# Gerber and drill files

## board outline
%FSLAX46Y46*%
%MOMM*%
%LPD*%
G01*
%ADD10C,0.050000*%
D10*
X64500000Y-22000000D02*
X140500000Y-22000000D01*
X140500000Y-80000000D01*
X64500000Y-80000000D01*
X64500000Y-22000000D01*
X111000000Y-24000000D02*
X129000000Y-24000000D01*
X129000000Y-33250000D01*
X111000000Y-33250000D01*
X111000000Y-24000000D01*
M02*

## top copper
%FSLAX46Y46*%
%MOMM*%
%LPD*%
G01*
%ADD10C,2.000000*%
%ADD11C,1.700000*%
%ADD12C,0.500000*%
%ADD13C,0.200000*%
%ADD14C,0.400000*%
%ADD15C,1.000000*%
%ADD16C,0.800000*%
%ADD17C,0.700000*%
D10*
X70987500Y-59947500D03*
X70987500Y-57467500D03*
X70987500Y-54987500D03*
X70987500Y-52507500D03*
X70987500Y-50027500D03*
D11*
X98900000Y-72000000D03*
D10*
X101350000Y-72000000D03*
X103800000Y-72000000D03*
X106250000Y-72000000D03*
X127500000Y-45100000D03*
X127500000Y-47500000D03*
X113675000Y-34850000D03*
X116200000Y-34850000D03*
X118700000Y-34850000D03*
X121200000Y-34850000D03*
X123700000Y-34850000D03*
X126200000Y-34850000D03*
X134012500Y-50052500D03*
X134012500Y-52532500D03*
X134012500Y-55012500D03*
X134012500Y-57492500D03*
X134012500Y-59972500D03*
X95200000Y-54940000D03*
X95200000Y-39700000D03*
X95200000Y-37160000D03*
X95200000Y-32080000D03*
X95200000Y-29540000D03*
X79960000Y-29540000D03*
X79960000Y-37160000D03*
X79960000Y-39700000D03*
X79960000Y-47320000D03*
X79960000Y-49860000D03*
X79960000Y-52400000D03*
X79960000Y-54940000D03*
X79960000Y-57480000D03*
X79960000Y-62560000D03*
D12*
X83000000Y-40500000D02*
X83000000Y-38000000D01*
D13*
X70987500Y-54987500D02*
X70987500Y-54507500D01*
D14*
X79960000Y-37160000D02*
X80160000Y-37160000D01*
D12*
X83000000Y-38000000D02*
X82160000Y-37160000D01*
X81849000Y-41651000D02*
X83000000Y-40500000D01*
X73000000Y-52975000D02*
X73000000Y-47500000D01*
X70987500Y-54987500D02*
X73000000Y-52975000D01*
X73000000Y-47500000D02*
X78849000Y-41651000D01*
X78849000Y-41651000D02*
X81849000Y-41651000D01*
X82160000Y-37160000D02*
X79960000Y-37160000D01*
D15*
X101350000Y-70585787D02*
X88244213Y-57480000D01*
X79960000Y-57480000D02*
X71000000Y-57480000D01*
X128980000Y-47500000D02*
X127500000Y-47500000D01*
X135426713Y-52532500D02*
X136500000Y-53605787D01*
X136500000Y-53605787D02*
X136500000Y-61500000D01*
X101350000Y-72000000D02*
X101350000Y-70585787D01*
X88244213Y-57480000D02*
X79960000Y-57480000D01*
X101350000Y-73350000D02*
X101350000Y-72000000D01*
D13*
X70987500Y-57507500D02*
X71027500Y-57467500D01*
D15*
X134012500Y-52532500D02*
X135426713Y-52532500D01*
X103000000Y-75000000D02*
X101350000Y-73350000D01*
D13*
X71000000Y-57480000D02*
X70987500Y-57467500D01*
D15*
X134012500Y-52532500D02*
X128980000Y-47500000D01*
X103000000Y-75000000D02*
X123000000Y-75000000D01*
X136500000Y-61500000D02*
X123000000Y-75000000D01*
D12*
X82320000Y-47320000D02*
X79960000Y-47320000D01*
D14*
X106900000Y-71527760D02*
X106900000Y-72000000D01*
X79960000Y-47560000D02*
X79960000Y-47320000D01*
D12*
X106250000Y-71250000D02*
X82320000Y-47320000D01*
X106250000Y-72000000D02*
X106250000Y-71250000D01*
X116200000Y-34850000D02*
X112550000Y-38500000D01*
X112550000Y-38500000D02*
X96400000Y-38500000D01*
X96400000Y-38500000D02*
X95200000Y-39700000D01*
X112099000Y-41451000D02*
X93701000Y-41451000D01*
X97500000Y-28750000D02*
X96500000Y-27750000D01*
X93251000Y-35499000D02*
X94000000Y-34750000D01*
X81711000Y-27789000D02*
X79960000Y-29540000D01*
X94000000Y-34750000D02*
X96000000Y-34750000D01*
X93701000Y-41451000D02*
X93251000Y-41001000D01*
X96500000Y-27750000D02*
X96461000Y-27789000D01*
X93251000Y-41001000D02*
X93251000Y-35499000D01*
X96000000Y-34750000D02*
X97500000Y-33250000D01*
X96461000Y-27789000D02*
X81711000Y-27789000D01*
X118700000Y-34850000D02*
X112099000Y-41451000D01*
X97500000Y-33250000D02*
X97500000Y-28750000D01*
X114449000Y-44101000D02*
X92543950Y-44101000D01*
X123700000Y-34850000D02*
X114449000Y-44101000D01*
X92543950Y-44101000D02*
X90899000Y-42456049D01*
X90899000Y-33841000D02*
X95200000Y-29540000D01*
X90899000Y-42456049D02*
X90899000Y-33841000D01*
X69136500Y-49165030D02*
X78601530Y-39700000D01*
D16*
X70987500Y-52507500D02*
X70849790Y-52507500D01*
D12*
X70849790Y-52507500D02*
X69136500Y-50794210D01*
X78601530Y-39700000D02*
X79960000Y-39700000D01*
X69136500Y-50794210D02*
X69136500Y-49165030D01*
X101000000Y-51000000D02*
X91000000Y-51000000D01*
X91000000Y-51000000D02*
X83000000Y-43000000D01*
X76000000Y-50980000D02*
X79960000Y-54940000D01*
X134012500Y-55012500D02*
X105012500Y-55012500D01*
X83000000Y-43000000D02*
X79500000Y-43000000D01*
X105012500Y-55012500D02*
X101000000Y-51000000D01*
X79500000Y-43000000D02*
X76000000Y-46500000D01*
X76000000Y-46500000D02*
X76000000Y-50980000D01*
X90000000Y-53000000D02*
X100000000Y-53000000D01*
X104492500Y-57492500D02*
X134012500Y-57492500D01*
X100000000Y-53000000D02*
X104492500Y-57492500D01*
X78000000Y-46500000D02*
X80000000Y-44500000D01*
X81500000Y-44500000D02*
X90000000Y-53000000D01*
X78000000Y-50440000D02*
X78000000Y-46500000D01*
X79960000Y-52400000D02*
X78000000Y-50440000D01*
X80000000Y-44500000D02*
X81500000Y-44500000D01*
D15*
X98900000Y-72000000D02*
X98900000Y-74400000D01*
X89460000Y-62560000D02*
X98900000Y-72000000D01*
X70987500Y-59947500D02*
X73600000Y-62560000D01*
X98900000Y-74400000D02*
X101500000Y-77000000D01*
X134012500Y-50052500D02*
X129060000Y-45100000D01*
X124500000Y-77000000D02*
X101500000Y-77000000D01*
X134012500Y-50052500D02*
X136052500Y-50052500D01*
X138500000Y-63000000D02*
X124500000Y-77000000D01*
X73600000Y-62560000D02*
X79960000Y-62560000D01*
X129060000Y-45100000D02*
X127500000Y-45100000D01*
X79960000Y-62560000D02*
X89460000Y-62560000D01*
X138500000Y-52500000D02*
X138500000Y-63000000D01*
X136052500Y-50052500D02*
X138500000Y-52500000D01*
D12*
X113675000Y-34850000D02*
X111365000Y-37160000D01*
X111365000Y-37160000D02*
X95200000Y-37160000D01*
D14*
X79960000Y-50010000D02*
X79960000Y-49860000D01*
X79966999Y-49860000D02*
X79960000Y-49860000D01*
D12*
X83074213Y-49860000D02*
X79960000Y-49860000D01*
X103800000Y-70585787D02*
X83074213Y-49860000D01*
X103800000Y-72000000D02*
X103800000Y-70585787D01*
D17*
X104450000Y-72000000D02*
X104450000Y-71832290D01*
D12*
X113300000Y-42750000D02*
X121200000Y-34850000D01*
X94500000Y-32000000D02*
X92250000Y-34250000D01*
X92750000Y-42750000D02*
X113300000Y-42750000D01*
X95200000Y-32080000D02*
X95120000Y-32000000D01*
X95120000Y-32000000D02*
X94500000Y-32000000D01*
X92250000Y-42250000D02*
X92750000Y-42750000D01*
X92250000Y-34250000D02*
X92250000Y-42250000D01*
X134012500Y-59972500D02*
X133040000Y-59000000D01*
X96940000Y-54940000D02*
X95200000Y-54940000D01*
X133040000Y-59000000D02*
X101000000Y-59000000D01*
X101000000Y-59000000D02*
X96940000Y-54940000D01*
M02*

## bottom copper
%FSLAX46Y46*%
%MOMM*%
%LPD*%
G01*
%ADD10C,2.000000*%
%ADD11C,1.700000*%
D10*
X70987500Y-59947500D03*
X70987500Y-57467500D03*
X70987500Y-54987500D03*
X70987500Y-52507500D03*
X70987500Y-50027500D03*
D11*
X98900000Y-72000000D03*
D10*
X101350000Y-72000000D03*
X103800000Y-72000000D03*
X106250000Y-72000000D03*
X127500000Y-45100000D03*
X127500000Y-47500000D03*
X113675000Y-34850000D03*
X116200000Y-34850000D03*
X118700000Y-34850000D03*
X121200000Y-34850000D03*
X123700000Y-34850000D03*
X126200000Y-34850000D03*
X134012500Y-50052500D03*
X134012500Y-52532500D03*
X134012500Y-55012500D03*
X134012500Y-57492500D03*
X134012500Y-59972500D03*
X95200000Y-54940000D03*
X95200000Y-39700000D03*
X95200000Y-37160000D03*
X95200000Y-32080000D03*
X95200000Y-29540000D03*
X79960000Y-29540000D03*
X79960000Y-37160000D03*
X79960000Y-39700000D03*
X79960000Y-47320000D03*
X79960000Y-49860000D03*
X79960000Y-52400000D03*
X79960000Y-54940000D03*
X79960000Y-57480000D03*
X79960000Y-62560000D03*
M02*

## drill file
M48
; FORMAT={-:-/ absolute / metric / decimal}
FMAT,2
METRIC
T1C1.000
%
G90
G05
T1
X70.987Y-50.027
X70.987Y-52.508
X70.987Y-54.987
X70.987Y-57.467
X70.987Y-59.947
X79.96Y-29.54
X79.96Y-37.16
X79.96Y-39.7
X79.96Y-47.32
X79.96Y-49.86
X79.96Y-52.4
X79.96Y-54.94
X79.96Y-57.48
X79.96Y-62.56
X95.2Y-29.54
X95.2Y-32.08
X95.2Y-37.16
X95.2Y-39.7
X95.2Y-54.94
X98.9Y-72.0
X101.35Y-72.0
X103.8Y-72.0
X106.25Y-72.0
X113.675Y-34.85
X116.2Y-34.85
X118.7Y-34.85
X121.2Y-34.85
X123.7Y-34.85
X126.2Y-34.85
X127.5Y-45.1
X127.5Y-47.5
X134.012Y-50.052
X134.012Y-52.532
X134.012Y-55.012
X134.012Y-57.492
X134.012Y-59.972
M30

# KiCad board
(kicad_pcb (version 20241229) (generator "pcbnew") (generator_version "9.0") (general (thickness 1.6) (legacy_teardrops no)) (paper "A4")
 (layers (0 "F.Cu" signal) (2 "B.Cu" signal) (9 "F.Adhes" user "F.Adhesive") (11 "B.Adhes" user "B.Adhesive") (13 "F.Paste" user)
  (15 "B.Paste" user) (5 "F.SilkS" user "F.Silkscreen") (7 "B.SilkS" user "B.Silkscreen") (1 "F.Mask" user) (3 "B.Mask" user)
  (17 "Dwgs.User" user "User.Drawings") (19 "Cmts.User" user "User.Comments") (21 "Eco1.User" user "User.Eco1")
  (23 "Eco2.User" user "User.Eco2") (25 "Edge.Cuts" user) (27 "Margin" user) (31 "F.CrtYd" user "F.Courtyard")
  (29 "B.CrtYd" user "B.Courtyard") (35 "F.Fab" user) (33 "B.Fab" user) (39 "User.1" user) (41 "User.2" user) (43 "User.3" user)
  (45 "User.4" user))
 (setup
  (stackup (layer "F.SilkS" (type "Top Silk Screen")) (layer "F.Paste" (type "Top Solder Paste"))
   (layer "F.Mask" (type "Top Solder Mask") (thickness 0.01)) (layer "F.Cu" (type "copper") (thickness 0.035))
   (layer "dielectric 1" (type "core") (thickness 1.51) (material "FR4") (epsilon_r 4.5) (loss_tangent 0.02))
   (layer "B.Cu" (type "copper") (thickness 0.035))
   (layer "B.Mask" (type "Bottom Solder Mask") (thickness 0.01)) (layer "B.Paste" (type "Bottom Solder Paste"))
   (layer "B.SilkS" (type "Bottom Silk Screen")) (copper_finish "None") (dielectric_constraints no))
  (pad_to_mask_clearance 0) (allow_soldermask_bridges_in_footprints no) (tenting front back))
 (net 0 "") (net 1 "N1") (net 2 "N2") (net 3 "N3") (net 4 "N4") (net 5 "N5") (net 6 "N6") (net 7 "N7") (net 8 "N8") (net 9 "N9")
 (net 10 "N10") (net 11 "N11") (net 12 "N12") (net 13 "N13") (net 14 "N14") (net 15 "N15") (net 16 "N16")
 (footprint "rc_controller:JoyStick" (layer "F.Cu") (at 72.1875 61.1875 180)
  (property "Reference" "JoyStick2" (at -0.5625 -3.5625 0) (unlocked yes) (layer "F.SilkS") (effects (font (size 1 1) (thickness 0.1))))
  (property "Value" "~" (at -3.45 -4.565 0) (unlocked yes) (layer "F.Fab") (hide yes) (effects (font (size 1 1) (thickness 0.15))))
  (pad "1" thru_hole circle (at 1.2 1.24 180) (size 2 2) (drill 1) (layers "*.Cu" "*.Mask") (remove_unused_layers no) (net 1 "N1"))
  (pad "2" thru_hole circle (at 1.2 3.72 180) (size 2 2) (drill 1) (layers "*.Cu" "*.Mask") (remove_unused_layers no) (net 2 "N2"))
  (pad "3" thru_hole circle (at 1.2 6.2 180) (size 2 2) (drill 1) (layers "*.Cu" "*.Mask") (remove_unused_layers no) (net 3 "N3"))
  (pad "4" thru_hole circle (at 1.2 8.68 180) (size 2 2) (drill 1) (layers "*.Cu" "*.Mask") (remove_unused_layers no) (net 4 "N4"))
  (pad "5" thru_hole circle (at 1.2 11.16 180) (size 2 2) (drill 1) (layers "*.Cu" "*.Mask") (remove_unused_layers no) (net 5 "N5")))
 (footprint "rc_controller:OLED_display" (layer "F.Cu") (at 97.675 73.2 90)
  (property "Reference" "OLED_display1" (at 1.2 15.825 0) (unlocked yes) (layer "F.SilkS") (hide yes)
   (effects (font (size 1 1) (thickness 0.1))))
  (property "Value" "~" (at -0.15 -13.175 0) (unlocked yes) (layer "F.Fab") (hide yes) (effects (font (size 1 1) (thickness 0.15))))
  (pad "1" thru_hole circle (at 1.2 1.225 90) (size 1.7 1.7) (drill 1) (layers "*.Cu" "*.Mask") (remove_unused_layers no) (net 1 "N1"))
  (pad "2" thru_hole circle (at 1.2 3.675 90) (size 2 2) (drill 1) (layers "*.Cu" "*.Mask") (remove_unused_layers no) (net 2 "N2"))
  (pad "3" thru_hole circle (at 1.2 6.125 90) (size 2 2) (drill 1) (layers "*.Cu" "F.Mask") (remove_unused_layers no) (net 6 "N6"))
  (pad "4" thru_hole circle (at 1.2 8.575 90) (size 2 2) (drill 1) (layers "*.Cu" "*.Mask") (remove_unused_layers no) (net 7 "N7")))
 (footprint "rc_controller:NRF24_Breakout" (layer "F.Cu") (at 110.65 24.1)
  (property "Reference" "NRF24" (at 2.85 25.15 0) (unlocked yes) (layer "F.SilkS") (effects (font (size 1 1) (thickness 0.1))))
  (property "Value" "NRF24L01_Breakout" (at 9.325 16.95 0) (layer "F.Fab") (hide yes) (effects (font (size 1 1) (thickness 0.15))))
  (pad "1" thru_hole circle (at 16.85 21) (size 2 2) (drill 1) (layers "*.Cu" "*.Mask") (remove_unused_layers no) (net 1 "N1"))
  (pad "2" thru_hole circle (at 16.85 23.4) (size 2 2) (drill 1) (layers "*.Cu" "*.Mask") (remove_unused_layers no) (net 2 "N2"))
  (pad "3" thru_hole circle (at 3.025 10.75) (size 2 2) (drill 1) (layers "*.Cu" "*.Mask") (remove_unused_layers no) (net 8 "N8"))
  (pad "4" thru_hole circle (at 5.55 10.75) (size 2 2) (drill 1) (layers "*.Cu" "*.Mask") (remove_unused_layers no) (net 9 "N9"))
  (pad "5" thru_hole circle (at 8.05 10.75) (size 2 2) (drill 1) (layers "*.Cu" "*.Mask") (remove_unused_layers no) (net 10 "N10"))
  (pad "6" thru_hole circle (at 10.55 10.75) (size 2 2) (drill 1) (layers "*.Cu" "*.Mask") (remove_unused_layers no) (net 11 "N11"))
  (pad "7" thru_hole circle (at 13.05 10.75) (size 2 2) (drill 1) (layers "*.Cu" "*.Mask") (remove_unused_layers no) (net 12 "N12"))
  (pad "8" thru_hole circle (at 15.55 10.75) (size 2 2) (drill 1) (layers "*.Cu" "*.Mask") (remove_unused_layers no) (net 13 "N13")))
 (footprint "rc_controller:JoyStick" (layer "F.Cu") (at 132.8125 48.8125)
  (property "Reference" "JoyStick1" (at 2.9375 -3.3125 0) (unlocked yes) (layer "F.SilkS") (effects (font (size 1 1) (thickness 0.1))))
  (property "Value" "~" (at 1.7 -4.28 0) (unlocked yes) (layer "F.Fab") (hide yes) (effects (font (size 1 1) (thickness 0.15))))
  (pad "1" thru_hole circle (at 1.2 1.24) (size 2 2) (drill 1) (layers "*.Cu" "*.Mask") (remove_unused_layers no) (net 1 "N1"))
  (pad "2" thru_hole circle (at 1.2 3.72) (size 2 2) (drill 1) (layers "*.Cu" "*.Mask") (remove_unused_layers no) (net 2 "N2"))
  (pad "3" thru_hole circle (at 1.2 6.2) (size 2 2) (drill 1) (layers "*.Cu" "*.Mask") (remove_unused_layers no) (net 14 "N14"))
  (pad "4" thru_hole circle (at 1.2 8.68) (size 2 2) (drill 1) (layers "*.Cu" "*.Mask") (remove_unused_layers no) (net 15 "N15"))
  (pad "5" thru_hole circle (at 1.2 11.16) (size 2 2) (drill 1) (layers "*.Cu" "*.Mask") (remove_unused_layers no) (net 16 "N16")))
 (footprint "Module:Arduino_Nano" (layer "F.Cu") (at 80 27)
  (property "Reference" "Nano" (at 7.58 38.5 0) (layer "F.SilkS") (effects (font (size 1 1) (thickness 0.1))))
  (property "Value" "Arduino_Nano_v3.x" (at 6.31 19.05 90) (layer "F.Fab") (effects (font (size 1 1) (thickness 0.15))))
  (pad "5" thru_hole circle (at 15.2 27.94 180) (size 2 2) (drill 1) (layers "*.Cu" "*.Mask") (remove_unused_layers no) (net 16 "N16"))
  (pad "11" thru_hole circle (at 15.2 12.7 180) (size 2 2) (drill 1) (layers "*.Cu" "*.Mask") (remove_unused_layers no) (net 9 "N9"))
  (pad "12" thru_hole circle (at 15.2 10.16 180) (size 2 2) (drill 1) (layers "*.Cu" "*.Mask") (remove_unused_layers no) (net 8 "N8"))
  (pad "14" thru_hole circle (at 15.2 5.08 180) (size 2 2) (drill 1) (layers "*.Cu" "*.Mask") (remove_unused_layers no) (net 11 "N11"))
  (pad "15" thru_hole circle (at 15.2 2.54 180) (size 2 2) (drill 1) (layers "*.Cu" "*.Mask") (remove_unused_layers no) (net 12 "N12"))
  (pad "16" thru_hole circle (at -0.04 2.54 180) (size 2 2) (drill 1) (layers "*.Cu" "*.Mask") (remove_unused_layers no) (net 10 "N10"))
  (pad "19" thru_hole circle (at -0.04 10.16 180) (size 2 2) (drill 1) (layers "*.Cu" "*.Mask") (remove_unused_layers no) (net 3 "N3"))
  (pad "20" thru_hole circle (at -0.04 12.7 180) (size 2 2) (drill 1) (layers "*.Cu" "*.Mask") (remove_unused_layers no) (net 4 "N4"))
  (pad "23" thru_hole circle (at -0.04 20.32 180) (size 2 2) (drill 1) (layers "*.Cu" "*.Mask") (remove_unused_layers no) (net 7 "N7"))
  (pad "24" thru_hole circle (at -0.04 22.86 180) (size 2 2) (drill 1) (layers "*.Cu" "*.Mask") (remove_unused_layers no) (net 6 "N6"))
  (pad "25" thru_hole circle (at -0.04 25.4 180) (size 2 2) (drill 1) (layers "*.Cu" "*.Mask") (remove_unused_layers no) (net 15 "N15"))
  (pad "26" thru_hole circle (at -0.04 27.94 180) (size 2 2) (drill 1) (layers "*.Cu" "*.Mask") (remove_unused_layers no) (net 14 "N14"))
  (pad "27" thru_hole circle (at -0.04 30.48 180) (size 2 2) (drill 1) (layers "*.Cu" "*.Mask") (remove_unused_layers no) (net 2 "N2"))
  (pad "29" thru_hole circle (at -0.04 35.56 180) (size 2 2) (drill 1) (layers "*.Cu" "*.Mask") (remove_unused_layers no) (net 1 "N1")))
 (gr_rect (start 64.5 22) (end 140.5 80) (stroke (width 0.05) (type default)) (fill no) (layer "Edge.Cuts"))
 (gr_rect (start 111 24) (end 129 33.25) (stroke (width 0.05) (type solid)) (fill no) (layer "Edge.Cuts"))
 (segment (start 83 40.5) (end 83 38) (width 0.5) (layer "F.Cu") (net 3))
 (segment (start 70.9875 54.9875) (end 70.9875 54.5075) (width 0.2) (layer "F.Cu") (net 3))
 (segment (start 79.96 37.16) (end 80.16 37.16) (width 0.4) (layer "F.Cu") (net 3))
 (segment (start 83 38) (end 82.16 37.16) (width 0.5) (layer "F.Cu") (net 3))
 (segment (start 81.849 41.651) (end 83 40.5) (width 0.5) (layer "F.Cu") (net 3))
 (segment (start 73 52.975) (end 73 47.5) (width 0.5) (layer "F.Cu") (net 3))
 (segment (start 70.9875 54.9875) (end 73 52.975) (width 0.5) (layer "F.Cu") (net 3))
 (segment (start 73 47.5) (end 78.849 41.651) (width 0.5) (layer "F.Cu") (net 3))
 (segment (start 78.849 41.651) (end 81.849 41.651) (width 0.5) (layer "F.Cu") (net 3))
 (segment (start 82.16 37.16) (end 79.96 37.16) (width 0.5) (layer "F.Cu") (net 3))
 (segment (start 101.35 70.585787) (end 88.244213 57.48) (width 1) (layer "F.Cu") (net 2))
 (segment (start 79.96 57.48) (end 71 57.48) (width 1) (layer "F.Cu") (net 2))
 (segment (start 128.98 47.5) (end 127.5 47.5) (width 1) (layer "F.Cu") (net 2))
 (segment (start 135.426713 52.5325) (end 136.5 53.605787) (width 1) (layer "F.Cu") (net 2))
 (segment (start 136.5 53.605787) (end 136.5 61.5) (width 1) (layer "F.Cu") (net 2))
 (segment (start 101.35 72) (end 101.35 70.585787) (width 1) (layer "F.Cu") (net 2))
 (segment (start 88.244213 57.48) (end 79.96 57.48) (width 1) (layer "F.Cu") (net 2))
 (segment (start 101.35 73.35) (end 101.35 72) (width 1) (layer "F.Cu") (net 2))
 (segment (start 70.9875 57.5075) (end 71.0275 57.4675) (width 0.2) (layer "F.Cu") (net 2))
 (segment (start 134.0125 52.5325) (end 135.426713 52.5325) (width 1) (layer "F.Cu") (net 2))
 (segment (start 103 75) (end 101.35 73.35) (width 1) (layer "F.Cu") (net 2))
 (segment (start 71 57.48) (end 70.9875 57.4675) (width 0.2) (layer "F.Cu") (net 2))
 (segment (start 134.0125 52.5325) (end 128.98 47.5) (width 1) (layer "F.Cu") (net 2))
 (segment (start 103 75) (end 123 75) (width 1) (layer "F.Cu") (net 2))
 (segment (start 136.5 61.5) (end 123 75) (width 1) (layer "F.Cu") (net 2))
 (segment (start 82.32 47.32) (end 79.96 47.32) (width 0.5) (layer "F.Cu") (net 7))
 (segment (start 106.9 71.52776) (end 106.9 72) (width 0.4) (layer "F.Cu") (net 7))
 (segment (start 79.96 47.56) (end 79.96 47.32) (width 0.4) (layer "F.Cu") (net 7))
 (segment (start 106.25 71.25) (end 82.32 47.32) (width 0.5) (layer "F.Cu") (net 7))
 (segment (start 106.25 72) (end 106.25 71.25) (width 0.5) (layer "F.Cu") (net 7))
 (segment (start 116.2 34.85) (end 112.55 38.5) (width 0.5) (layer "F.Cu") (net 9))
 (segment (start 112.55 38.5) (end 96.4 38.5) (width 0.5) (layer "F.Cu") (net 9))
 (segment (start 96.4 38.5) (end 95.2 39.7) (width 0.5) (layer "F.Cu") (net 9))
 (segment (start 112.099 41.451) (end 93.701 41.451) (width 0.5) (layer "F.Cu") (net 10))
 (segment (start 97.5 28.75) (end 96.5 27.75) (width 0.5) (layer "F.Cu") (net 10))
 (segment (start 93.251 35.499) (end 94 34.75) (width 0.5) (layer "F.Cu") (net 10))
 (segment (start 81.711 27.789) (end 79.96 29.54) (width 0.5) (layer "F.Cu") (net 10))
 (segment (start 94 34.75) (end 96 34.75) (width 0.5) (layer "F.Cu") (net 10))
 (segment (start 93.701 41.451) (end 93.251 41.001) (width 0.5) (layer "F.Cu") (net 10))
 (segment (start 96.5 27.75) (end 96.461 27.789) (width 0.5) (layer "F.Cu") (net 10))
 (segment (start 93.251 41.001) (end 93.251 35.499) (width 0.5) (layer "F.Cu") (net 10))
 (segment (start 96 34.75) (end 97.5 33.25) (width 0.5) (layer "F.Cu") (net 10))
 (segment (start 96.461 27.789) (end 81.711 27.789) (width 0.5) (layer "F.Cu") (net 10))
 (segment (start 118.7 34.85) (end 112.099 41.451) (width 0.5) (layer "F.Cu") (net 10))
 (segment (start 97.5 33.25) (end 97.5 28.75) (width 0.5) (layer "F.Cu") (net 10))
 (segment (start 114.449 44.101) (end 92.54395 44.101) (width 0.5) (layer "F.Cu") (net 12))
 (segment (start 123.7 34.85) (end 114.449 44.101) (width 0.5) (layer "F.Cu") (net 12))
 (segment (start 92.54395 44.101) (end 90.899 42.456049) (width 0.5) (layer "F.Cu") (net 12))
 (segment (start 90.899 33.841) (end 95.2 29.54) (width 0.5) (layer "F.Cu") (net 12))
 (segment (start 90.899 42.456049) (end 90.899 33.841) (width 0.5) (layer "F.Cu") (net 12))
 (segment (start 69.1365 49.16503) (end 78.60153 39.7) (width 0.5) (layer "F.Cu") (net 4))
 (segment (start 70.9875 52.5075) (end 70.84979 52.5075) (width 0.8) (layer "F.Cu") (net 4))
 (segment (start 70.84979 52.5075) (end 69.1365 50.79421) (width 0.5) (layer "F.Cu") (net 4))
 (segment (start 78.60153 39.7) (end 79.96 39.7) (width 0.5) (layer "F.Cu") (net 4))
 (segment (start 69.1365 50.79421) (end 69.1365 49.16503) (width 0.5) (layer "F.Cu") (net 4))
 (segment (start 101 51) (end 91 51) (width 0.5) (layer "F.Cu") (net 14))
 (segment (start 91 51) (end 83 43) (width 0.5) (layer "F.Cu") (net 14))
 (segment (start 76 50.98) (end 79.96 54.94) (width 0.5) (layer "F.Cu") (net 14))
 (segment (start 134.0125 55.0125) (end 105.0125 55.0125) (width 0.5) (layer "F.Cu") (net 14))
 (segment (start 83 43) (end 79.5 43) (width 0.5) (layer "F.Cu") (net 14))
 (segment (start 105.0125 55.0125) (end 101 51) (width 0.5) (layer "F.Cu") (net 14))
 (segment (start 79.5 43) (end 76 46.5) (width 0.5) (layer "F.Cu") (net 14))
 (segment (start 76 46.5) (end 76 50.98) (width 0.5) (layer "F.Cu") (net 14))
 (segment (start 90 53) (end 100 53) (width 0.5) (layer "F.Cu") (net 15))
 (segment (start 104.4925 57.4925) (end 134.0125 57.4925) (width 0.5) (layer "F.Cu") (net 15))
 (segment (start 100 53) (end 104.4925 57.4925) (width 0.5) (layer "F.Cu") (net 15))
 (segment (start 78 46.5) (end 80 44.5) (width 0.5) (layer "F.Cu") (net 15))
 (segment (start 81.5 44.5) (end 90 53) (width 0.5) (layer "F.Cu") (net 15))
 (segment (start 78 50.44) (end 78 46.5) (width 0.5) (layer "F.Cu") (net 15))
 (segment (start 79.96 52.4) (end 78 50.44) (width 0.5) (layer "F.Cu") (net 15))
 (segment (start 80 44.5) (end 81.5 44.5) (width 0.5) (layer "F.Cu") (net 15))
 (segment (start 98.9 72) (end 98.9 74.4) (width 1) (layer "F.Cu") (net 1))
 (segment (start 89.46 62.56) (end 98.9 72) (width 1) (layer "F.Cu") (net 1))
 (segment (start 70.9875 59.9475) (end 73.6 62.56) (width 1) (layer "F.Cu") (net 1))
 (segment (start 98.9 74.4) (end 101.5 77) (width 1) (layer "F.Cu") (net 1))
 (segment (start 134.0125 50.0525) (end 129.06 45.1) (width 1) (layer "F.Cu") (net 1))
 (segment (start 124.5 77) (end 101.5 77) (width 1) (layer "F.Cu") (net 1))
 (segment (start 134.0125 50.0525) (end 136.0525 50.0525) (width 1) (layer "F.Cu") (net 1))
 (segment (start 138.5 63) (end 124.5 77) (width 1) (layer "F.Cu") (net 1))
 (segment (start 73.6 62.56) (end 79.96 62.56) (width 1) (layer "F.Cu") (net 1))
 (segment (start 129.06 45.1) (end 127.5 45.1) (width 1) (layer "F.Cu") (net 1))
 (segment (start 79.96 62.56) (end 89.46 62.56) (width 1) (layer "F.Cu") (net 1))
 (segment (start 138.5 52.5) (end 138.5 63) (width 1) (layer "F.Cu") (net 1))
 (segment (start 136.0525 50.0525) (end 138.5 52.5) (width 1) (layer "F.Cu") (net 1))
 (segment (start 113.675 34.85) (end 111.365 37.16) (width 0.5) (layer "F.Cu") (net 8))
 (segment (start 111.365 37.16) (end 95.2 37.16) (width 0.5) (layer "F.Cu") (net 8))
 (segment (start 79.96 50.01) (end 79.96 49.86) (width 0.4) (layer "F.Cu") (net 6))
 (segment (start 79.966999 49.86) (end 79.96 49.86) (width 0.4) (layer "F.Cu") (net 6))
 (segment (start 83.074213 49.86) (end 79.96 49.86) (width 0.5) (layer "F.Cu") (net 6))
 (segment (start 103.8 70.585787) (end 83.074213 49.86) (width 0.5) (layer "F.Cu") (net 6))
 (segment (start 103.8 72) (end 103.8 70.585787) (width 0.5) (layer "F.Cu") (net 6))
 (segment (start 104.45 72) (end 104.45 71.83229) (width 0.7) (layer "F.Cu") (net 6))
 (segment (start 113.3 42.75) (end 121.2 34.85) (width 0.5) (layer "F.Cu") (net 11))
 (segment (start 94.5 32) (end 92.25 34.25) (width 0.5) (layer "F.Cu") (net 11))
 (segment (start 92.75 42.75) (end 113.3 42.75) (width 0.5) (layer "F.Cu") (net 11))
 (segment (start 95.2 32.08) (end 95.12 32) (width 0.5) (layer "F.Cu") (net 11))
 (segment (start 95.12 32) (end 94.5 32) (width 0.5) (layer "F.Cu") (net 11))
 (segment (start 92.25 42.25) (end 92.75 42.75) (width 0.5) (layer "F.Cu") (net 11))
 (segment (start 92.25 34.25) (end 92.25 42.25) (width 0.5) (layer "F.Cu") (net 11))
 (segment (start 134.0125 59.9725) (end 133.04 59) (width 0.5) (layer "F.Cu") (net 16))
 (segment (start 96.94 54.94) (end 95.2 54.94) (width 0.5) (layer "F.Cu") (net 16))
 (segment (start 133.04 59) (end 101 59) (width 0.5) (layer "F.Cu") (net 16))
 (segment (start 101 59) (end 96.94 54.94) (width 0.5) (layer "F.Cu") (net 16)))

